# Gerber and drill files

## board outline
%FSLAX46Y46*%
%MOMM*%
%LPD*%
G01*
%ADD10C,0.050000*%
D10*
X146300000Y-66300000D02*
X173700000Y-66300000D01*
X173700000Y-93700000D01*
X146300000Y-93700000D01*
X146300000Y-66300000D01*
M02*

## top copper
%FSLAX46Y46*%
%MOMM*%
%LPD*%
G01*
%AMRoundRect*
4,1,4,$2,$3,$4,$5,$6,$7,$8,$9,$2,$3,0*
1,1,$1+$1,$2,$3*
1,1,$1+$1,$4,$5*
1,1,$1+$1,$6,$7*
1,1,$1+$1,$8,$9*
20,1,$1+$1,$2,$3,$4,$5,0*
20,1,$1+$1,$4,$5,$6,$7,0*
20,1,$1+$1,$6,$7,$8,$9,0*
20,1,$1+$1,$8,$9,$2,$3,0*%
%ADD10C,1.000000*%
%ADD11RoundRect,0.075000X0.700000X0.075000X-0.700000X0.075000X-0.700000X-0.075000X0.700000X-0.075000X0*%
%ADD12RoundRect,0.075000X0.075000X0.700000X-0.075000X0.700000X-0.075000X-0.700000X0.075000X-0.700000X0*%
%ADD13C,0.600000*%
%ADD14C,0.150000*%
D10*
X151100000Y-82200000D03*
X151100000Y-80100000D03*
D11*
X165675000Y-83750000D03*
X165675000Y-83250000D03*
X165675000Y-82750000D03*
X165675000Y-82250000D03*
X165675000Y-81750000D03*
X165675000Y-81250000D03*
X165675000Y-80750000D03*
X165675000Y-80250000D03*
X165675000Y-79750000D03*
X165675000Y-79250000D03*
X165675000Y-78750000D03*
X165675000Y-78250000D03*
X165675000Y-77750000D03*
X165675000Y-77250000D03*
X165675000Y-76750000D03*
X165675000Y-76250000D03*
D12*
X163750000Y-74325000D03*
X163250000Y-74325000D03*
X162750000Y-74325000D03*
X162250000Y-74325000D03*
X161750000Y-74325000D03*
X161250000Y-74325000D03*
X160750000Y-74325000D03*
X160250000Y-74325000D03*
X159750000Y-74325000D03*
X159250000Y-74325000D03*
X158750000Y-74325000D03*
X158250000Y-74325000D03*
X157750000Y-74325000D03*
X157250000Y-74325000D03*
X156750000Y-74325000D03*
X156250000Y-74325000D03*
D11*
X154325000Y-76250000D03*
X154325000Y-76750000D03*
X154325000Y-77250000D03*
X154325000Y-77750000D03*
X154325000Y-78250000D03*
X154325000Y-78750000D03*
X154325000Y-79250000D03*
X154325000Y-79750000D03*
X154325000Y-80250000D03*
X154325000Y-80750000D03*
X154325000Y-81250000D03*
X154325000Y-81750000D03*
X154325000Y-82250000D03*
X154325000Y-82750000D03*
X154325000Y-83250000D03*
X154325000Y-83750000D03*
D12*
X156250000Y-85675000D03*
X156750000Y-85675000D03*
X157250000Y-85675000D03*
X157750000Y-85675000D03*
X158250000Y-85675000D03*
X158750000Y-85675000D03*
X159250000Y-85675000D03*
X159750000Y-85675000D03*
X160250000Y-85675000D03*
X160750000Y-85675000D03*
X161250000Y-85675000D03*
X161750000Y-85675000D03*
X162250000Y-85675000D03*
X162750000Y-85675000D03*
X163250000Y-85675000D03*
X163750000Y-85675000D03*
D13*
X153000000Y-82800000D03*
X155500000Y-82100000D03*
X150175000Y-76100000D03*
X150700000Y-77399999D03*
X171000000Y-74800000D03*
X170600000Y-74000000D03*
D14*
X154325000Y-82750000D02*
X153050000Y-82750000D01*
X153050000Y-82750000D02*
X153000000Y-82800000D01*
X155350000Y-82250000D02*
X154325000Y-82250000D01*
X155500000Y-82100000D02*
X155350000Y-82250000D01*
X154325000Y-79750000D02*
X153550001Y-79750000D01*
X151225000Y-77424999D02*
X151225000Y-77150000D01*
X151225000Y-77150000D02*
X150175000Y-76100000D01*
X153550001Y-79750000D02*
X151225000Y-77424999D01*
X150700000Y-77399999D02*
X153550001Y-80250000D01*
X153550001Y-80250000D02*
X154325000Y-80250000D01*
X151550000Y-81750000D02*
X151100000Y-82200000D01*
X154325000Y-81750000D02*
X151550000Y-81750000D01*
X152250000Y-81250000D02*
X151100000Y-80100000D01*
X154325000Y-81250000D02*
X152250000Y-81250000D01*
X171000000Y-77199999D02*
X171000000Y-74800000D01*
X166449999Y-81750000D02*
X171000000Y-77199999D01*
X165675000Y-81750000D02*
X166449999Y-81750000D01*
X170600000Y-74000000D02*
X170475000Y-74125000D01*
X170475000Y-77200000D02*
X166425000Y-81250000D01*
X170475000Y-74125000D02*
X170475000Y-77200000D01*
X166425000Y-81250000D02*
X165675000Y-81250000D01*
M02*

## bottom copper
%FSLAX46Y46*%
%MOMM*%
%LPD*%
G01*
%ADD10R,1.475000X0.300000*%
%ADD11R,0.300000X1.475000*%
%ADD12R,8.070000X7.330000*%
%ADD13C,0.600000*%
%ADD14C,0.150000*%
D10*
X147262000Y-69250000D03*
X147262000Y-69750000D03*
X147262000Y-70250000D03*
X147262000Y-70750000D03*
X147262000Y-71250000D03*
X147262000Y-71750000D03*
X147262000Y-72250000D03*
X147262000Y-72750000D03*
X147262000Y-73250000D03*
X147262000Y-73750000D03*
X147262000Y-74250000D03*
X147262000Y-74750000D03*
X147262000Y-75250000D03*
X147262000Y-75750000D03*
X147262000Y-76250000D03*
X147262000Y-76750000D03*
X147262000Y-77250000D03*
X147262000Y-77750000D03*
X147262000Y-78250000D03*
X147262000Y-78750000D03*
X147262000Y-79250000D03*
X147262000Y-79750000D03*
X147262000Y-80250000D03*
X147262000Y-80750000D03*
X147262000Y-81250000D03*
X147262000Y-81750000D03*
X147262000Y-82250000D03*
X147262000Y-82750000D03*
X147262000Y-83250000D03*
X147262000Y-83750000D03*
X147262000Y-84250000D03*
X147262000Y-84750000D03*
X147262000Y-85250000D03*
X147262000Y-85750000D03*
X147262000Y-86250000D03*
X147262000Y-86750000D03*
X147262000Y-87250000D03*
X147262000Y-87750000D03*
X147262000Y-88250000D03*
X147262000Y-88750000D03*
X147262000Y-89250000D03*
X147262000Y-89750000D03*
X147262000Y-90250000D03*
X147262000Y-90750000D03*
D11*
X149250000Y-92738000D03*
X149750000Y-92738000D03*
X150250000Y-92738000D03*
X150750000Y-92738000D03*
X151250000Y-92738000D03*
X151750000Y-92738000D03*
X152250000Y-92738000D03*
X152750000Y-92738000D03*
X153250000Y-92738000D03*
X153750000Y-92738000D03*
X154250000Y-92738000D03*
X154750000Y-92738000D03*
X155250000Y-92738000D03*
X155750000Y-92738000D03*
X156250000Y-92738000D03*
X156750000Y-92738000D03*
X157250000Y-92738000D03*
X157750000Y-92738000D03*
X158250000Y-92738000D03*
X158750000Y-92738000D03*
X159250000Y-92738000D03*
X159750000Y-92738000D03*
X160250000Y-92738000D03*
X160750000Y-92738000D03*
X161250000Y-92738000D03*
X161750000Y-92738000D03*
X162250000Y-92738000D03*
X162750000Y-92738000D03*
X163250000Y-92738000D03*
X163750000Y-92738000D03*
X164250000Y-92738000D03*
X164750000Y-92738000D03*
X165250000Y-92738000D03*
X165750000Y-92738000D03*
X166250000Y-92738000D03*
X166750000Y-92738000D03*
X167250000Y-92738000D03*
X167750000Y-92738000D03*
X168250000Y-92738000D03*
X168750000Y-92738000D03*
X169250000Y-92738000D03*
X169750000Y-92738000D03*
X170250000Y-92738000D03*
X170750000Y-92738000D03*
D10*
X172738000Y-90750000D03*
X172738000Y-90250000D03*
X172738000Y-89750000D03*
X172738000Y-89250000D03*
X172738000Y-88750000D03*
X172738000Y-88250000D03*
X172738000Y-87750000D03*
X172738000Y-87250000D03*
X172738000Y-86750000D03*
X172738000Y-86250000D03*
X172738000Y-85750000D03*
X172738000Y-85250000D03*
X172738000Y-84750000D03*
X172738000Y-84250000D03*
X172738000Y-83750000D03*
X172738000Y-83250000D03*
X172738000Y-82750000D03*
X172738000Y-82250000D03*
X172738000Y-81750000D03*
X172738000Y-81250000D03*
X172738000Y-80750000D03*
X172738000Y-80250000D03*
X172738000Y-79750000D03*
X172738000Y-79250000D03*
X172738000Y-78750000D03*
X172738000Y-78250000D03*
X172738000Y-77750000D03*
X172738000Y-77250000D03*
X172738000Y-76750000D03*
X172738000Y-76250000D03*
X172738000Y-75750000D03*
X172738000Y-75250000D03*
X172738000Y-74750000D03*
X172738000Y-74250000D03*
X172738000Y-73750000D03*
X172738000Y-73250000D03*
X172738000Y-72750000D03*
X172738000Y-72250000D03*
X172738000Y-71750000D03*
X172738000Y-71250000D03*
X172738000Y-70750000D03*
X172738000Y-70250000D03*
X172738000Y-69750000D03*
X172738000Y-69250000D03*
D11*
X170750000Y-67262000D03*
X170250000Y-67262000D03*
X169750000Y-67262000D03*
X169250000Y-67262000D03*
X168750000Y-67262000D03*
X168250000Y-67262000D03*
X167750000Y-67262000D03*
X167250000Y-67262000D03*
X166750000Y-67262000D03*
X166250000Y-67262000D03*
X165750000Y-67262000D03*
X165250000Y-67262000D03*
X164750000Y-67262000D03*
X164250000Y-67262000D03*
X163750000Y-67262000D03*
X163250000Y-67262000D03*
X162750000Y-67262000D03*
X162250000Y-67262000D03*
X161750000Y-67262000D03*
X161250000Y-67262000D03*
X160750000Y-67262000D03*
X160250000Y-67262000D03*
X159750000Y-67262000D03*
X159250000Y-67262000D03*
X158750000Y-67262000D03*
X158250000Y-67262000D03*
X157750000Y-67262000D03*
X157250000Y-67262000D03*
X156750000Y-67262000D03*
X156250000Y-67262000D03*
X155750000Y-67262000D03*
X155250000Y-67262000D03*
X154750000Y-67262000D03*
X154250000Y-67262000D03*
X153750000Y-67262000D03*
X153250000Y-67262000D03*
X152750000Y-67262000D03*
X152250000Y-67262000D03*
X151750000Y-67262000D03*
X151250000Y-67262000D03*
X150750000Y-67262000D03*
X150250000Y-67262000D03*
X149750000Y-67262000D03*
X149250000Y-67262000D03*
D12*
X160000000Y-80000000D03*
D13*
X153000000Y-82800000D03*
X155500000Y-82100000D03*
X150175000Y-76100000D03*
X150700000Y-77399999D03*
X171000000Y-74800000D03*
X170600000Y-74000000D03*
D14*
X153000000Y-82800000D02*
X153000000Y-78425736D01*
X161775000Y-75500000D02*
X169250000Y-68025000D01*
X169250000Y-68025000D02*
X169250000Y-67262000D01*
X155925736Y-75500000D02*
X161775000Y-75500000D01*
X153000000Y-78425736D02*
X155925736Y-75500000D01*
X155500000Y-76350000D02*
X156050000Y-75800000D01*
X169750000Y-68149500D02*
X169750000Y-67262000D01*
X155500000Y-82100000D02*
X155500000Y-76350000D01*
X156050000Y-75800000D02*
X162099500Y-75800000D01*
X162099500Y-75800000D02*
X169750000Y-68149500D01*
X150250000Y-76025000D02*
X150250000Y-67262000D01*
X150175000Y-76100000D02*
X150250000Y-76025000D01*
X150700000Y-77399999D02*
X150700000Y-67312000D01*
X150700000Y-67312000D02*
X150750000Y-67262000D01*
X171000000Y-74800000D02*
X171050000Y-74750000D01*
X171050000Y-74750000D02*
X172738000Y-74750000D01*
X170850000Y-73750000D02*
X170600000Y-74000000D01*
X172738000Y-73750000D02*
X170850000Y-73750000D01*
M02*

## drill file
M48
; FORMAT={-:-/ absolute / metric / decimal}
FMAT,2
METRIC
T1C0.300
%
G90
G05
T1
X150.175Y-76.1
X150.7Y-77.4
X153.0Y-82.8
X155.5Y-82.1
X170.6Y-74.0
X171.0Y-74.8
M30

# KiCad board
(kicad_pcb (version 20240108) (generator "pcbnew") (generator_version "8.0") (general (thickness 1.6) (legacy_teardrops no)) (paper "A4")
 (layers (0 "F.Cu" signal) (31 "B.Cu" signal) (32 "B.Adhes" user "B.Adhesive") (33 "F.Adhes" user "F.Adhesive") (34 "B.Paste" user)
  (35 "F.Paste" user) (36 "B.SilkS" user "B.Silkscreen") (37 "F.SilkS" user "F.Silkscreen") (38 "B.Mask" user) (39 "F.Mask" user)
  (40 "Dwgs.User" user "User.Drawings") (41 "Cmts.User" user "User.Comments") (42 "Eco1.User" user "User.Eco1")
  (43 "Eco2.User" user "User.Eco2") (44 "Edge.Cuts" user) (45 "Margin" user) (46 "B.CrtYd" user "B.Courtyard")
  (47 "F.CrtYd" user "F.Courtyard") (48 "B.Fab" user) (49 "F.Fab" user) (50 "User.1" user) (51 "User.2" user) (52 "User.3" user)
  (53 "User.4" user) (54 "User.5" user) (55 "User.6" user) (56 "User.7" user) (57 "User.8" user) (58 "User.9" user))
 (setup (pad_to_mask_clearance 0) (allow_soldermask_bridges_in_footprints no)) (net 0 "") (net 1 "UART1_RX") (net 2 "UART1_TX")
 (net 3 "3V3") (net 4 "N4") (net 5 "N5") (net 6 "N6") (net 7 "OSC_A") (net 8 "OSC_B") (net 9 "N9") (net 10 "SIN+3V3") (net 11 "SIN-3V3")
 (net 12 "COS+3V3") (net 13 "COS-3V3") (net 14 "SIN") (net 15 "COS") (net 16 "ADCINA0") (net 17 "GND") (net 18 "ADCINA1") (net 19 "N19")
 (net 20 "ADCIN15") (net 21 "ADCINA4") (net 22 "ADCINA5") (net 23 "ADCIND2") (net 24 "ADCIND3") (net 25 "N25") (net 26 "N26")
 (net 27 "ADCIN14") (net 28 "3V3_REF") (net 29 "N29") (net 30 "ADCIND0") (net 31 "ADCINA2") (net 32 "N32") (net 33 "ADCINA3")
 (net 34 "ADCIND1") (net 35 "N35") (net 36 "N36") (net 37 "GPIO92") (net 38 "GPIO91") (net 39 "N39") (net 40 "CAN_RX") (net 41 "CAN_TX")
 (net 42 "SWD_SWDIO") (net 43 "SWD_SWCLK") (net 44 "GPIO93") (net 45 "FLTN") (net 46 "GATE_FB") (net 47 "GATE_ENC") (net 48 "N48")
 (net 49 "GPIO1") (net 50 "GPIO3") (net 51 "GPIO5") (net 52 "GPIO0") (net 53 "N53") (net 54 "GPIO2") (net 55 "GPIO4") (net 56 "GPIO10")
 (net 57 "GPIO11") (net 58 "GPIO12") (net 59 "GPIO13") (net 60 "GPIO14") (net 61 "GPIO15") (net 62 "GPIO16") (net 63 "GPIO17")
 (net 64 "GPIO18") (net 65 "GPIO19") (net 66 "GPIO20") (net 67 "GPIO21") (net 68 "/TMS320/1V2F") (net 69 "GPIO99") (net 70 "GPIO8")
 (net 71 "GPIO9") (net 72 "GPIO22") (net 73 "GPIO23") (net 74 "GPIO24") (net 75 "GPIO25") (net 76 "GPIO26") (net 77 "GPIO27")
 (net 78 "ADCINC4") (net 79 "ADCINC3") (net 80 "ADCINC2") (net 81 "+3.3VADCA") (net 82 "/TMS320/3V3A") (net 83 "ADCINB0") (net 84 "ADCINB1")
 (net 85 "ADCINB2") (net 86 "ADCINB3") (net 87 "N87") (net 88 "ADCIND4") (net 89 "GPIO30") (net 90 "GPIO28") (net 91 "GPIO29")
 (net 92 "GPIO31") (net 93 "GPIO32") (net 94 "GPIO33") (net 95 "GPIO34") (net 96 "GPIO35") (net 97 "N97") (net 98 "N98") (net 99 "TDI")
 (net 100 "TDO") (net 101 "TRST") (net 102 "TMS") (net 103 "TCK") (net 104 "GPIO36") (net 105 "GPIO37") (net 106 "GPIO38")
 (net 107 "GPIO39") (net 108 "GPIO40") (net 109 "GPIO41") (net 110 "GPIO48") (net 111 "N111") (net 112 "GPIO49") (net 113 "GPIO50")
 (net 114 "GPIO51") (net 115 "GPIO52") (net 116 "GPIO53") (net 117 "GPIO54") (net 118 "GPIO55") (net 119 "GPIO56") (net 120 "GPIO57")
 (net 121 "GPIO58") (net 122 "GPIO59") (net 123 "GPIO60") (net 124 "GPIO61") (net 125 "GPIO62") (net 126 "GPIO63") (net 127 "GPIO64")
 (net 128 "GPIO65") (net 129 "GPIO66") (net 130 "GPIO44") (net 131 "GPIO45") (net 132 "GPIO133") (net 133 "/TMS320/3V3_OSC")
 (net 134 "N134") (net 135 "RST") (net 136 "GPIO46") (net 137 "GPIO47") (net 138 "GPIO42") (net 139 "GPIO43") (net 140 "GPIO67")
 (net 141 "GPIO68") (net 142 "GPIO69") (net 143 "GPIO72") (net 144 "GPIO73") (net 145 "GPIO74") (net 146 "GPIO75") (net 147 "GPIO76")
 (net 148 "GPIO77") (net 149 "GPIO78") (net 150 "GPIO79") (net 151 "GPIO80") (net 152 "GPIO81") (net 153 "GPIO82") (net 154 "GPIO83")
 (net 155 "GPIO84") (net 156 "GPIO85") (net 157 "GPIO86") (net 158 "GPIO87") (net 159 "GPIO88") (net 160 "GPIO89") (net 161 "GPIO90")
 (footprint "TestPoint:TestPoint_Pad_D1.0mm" (layer "F.Cu") (at 151.1 82.2)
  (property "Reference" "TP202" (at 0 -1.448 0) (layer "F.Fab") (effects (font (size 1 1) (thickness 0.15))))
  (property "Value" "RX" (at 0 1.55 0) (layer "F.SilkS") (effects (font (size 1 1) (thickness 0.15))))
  (pad "1" smd circle (at 0 0) (size 1 1) (layers "F.Cu" "F.Mask") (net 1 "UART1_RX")))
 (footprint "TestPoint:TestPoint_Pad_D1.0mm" (layer "F.Cu") (at 151.1 80.1)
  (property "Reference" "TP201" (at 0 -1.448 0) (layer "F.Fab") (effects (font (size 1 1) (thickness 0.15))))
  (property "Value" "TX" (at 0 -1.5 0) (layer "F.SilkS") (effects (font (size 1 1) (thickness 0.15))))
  (pad "1" smd circle (at 0 0) (size 1 1) (layers "F.Cu" "F.Mask") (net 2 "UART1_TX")))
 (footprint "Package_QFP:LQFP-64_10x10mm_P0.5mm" (layer "F.Cu") (at 160 80 180)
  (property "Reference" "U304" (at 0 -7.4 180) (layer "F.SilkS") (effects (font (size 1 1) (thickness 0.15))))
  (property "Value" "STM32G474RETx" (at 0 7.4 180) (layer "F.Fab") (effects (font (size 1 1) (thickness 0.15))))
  (pad "1" smd roundrect (at -5.675 -3.75 180) (size 1.55 0.3) (layers "F.Cu" "F.Paste" "F.Mask") (roundrect_rratio 0.25) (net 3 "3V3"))
  (pad "2" smd roundrect (at -5.675 -3.25 180) (size 1.55 0.3) (layers "F.Cu" "F.Paste" "F.Mask") (roundrect_rratio 0.25) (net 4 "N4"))
  (pad "3" smd roundrect (at -5.675 -2.75 180) (size 1.55 0.3) (layers "F.Cu" "F.Paste" "F.Mask") (roundrect_rratio 0.25) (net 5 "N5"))
  (pad "4" smd roundrect (at -5.675 -2.25 180) (size 1.55 0.3) (layers "F.Cu" "F.Paste" "F.Mask") (roundrect_rratio 0.25) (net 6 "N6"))
  (pad "5" smd roundrect (at -5.675 -1.75 180) (size 1.55 0.3) (layers "F.Cu" "F.Paste" "F.Mask") (roundrect_rratio 0.25) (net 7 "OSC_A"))
  (pad "6" smd roundrect (at -5.675 -1.25 180) (size 1.55 0.3) (layers "F.Cu" "F.Paste" "F.Mask") (roundrect_rratio 0.25) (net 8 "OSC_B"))
  (pad "7" smd roundrect (at -5.675 -0.75 180) (size 1.55 0.3) (layers "F.Cu" "F.Paste" "F.Mask") (roundrect_rratio 0.25) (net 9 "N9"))
  (pad "8" smd roundrect (at -5.675 -0.25 180) (size 1.55 0.3) (layers "F.Cu" "F.Paste" "F.Mask") (roundrect_rratio 0.25) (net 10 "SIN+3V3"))
  (pad "9" smd roundrect (at -5.675 0.25 180) (size 1.55 0.3) (layers "F.Cu" "F.Paste" "F.Mask") (roundrect_rratio 0.25) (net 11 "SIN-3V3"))
  (pad "10" smd roundrect (at -5.675 0.75 180) (size 1.55 0.3) (layers "F.Cu" "F.Paste" "F.Mask") (roundrect_rratio 0.25) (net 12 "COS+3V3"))
  (pad "11" smd roundrect (at -5.675 1.25 180) (size 1.55 0.3) (layers "F.Cu" "F.Paste" "F.Mask") (roundrect_rratio 0.25) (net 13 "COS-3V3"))
  (pad "12" smd roundrect (at -5.675 1.75 180) (size 1.55 0.3) (layers "F.Cu" "F.Paste" "F.Mask") (roundrect_rratio 0.25) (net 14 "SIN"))
  (pad "13" smd roundrect (at -5.675 2.25 180) (size 1.55 0.3) (layers "F.Cu" "F.Paste" "F.Mask") (roundrect_rratio 0.25) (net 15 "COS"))
  (pad "14" smd roundrect (at -5.675 2.75 180) (size 1.55 0.3) (layers "F.Cu" "F.Paste" "F.Mask") (roundrect_rratio 0.25) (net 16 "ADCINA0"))
  (pad "15" smd roundrect (at -5.675 3.25 180) (size 1.55 0.3) (layers "F.Cu" "F.Paste" "F.Mask") (roundrect_rratio 0.25) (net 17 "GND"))
  (pad "16" smd roundrect (at -5.675 3.75 180) (size 1.55 0.3) (layers "F.Cu" "F.Paste" "F.Mask") (roundrect_rratio 0.25) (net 3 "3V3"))
  (pad "17" smd roundrect (at -3.75 5.675 180) (size 0.3 1.55) (layers "F.Cu" "F.Paste" "F.Mask") (roundrect_rratio 0.25) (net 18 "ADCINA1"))
  (pad "18" smd roundrect (at -3.25 5.675 180) (size 0.3 1.55) (layers "F.Cu" "F.Paste" "F.Mask") (roundrect_rratio 0.25) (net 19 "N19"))
  (pad "19" smd roundrect (at -2.75 5.675 180) (size 0.3 1.55) (layers "F.Cu" "F.Paste" "F.Mask") (roundrect_rratio 0.25) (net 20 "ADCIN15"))
  (pad "20" smd roundrect (at -2.25 5.675 180) (size 0.3 1.55) (layers "F.Cu" "F.Paste" "F.Mask") (roundrect_rratio 0.25) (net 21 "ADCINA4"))
  (pad "21" smd roundrect (at -1.75 5.675 180) (size 0.3 1.55) (layers "F.Cu" "F.Paste" "F.Mask") (roundrect_rratio 0.25) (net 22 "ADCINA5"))
  (pad "22" smd roundrect (at -1.25 5.675 180) (size 0.3 1.55) (layers "F.Cu" "F.Paste" "F.Mask") (roundrect_rratio 0.25) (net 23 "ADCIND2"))
  (pad "23" smd roundrect (at -0.75 5.675 180) (size 0.3 1.55) (layers "F.Cu" "F.Paste" "F.Mask") (roundrect_rratio 0.25) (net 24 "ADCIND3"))
  (pad "24" smd roundrect (at -0.25 5.675 180) (size 0.3 1.55) (layers "F.Cu" "F.Paste" "F.Mask") (roundrect_rratio 0.25) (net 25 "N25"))
  (pad "25" smd roundrect (at 0.25 5.675 180) (size 0.3 1.55) (layers "F.Cu" "F.Paste" "F.Mask") (roundrect_rratio 0.25) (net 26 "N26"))
  (pad "26" smd roundrect (at 0.75 5.675 180) (size 0.3 1.55) (layers "F.Cu" "F.Paste" "F.Mask") (roundrect_rratio 0.25) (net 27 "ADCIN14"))
  (pad "27" smd roundrect (at 1.25 5.675 180) (size 0.3 1.55) (layers "F.Cu" "F.Paste" "F.Mask") (roundrect_rratio 0.25) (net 17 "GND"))
  (pad "28" smd roundrect (at 1.75 5.675 180) (size 0.3 1.55) (layers "F.Cu" "F.Paste" "F.Mask") (roundrect_rratio 0.25) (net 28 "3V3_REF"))
  (pad "29" smd roundrect (at 2.25 5.675 180) (size 0.3 1.55) (layers "F.Cu" "F.Paste" "F.Mask") (roundrect_rratio 0.25) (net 3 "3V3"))
  (pad "30" smd roundrect (at 2.75 5.675 180) (size 0.3 1.55) (layers "F.Cu" "F.Paste" "F.Mask") (roundrect_rratio 0.25) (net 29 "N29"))
  (pad "31" smd roundrect (at 3.25 5.675 180) (size 0.3 1.55) (layers "F.Cu" "F.Paste" "F.Mask") (roundrect_rratio 0.25) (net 17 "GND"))
  (pad "32" smd roundrect (at 3.75 5.675 180) (size 0.3 1.55) (layers "F.Cu" "F.Paste" "F.Mask") (roundrect_rratio 0.25) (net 3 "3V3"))
  (pad "33" smd roundrect (at 5.675 3.75 180) (size 1.55 0.3) (layers "F.Cu" "F.Paste" "F.Mask") (roundrect_rratio 0.25) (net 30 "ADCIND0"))
  (pad "34" smd roundrect (at 5.675 3.25 180) (size 1.55 0.3) (layers "F.Cu" "F.Paste" "F.Mask") (roundrect_rratio 0.25) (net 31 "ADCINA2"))
  (pad "35" smd roundrect (at 5.675 2.75 180) (size 1.55 0.3) (layers "F.Cu" "F.Paste" "F.Mask") (roundrect_rratio 0.25) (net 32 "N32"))
  (pad "36" smd roundrect (at 5.675 2.25 180) (size 1.55 0.3) (layers "F.Cu" "F.Paste" "F.Mask") (roundrect_rratio 0.25) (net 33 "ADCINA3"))
  (pad "37" smd roundrect (at 5.675 1.75 180) (size 1.55 0.3) (layers "F.Cu" "F.Paste" "F.Mask") (roundrect_rratio 0.25) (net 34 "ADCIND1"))
  (pad "38" smd roundrect (at 5.675 1.25 180) (size 1.55 0.3) (layers "F.Cu" "F.Paste" "F.Mask") (roundrect_rratio 0.25) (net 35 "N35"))
  (pad "39" smd roundrect (at 5.675 0.75 180) (size 1.55 0.3) (layers "F.Cu" "F.Paste" "F.Mask") (roundrect_rratio 0.25) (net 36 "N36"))
  (pad "40" smd roundrect (at 5.675 0.25 180) (size 1.55 0.3) (layers "F.Cu" "F.Paste" "F.Mask") (roundrect_rratio 0.25) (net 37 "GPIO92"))
  (pad "41" smd roundrect (at 5.675 -0.25 180) (size 1.55 0.3) (layers "F.Cu" "F.Paste" "F.Mask") (roundrect_rratio 0.25) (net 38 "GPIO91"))
  (pad "42" smd roundrect (at 5.675 -0.75 180) (size 1.55 0.3) (layers "F.Cu" "F.Paste" "F.Mask") (roundrect_rratio 0.25) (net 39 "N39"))
  (pad "43" smd roundrect (at 5.675 -1.25 180) (size 1.55 0.3) (layers "F.Cu" "F.Paste" "F.Mask") (roundrect_rratio 0.25) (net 2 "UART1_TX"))
  (pad "44" smd roundrect (at 5.675 -1.75 180) (size 1.55 0.3) (layers "F.Cu" "F.Paste" "F.Mask") (roundrect_rratio 0.25) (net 1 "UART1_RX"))
  (pad "45" smd roundrect (at 5.675 -2.25 180) (size 1.55 0.3) (layers "F.Cu" "F.Paste" "F.Mask") (roundrect_rratio 0.25) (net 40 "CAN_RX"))
  (pad "46" smd roundrect (at 5.675 -2.75 180) (size 1.55 0.3) (layers "F.Cu" "F.Paste" "F.Mask") (roundrect_rratio 0.25) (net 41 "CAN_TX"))
  (pad "47" smd roundrect (at 5.675 -3.25 180) (size 1.55 0.3) (layers "F.Cu" "F.Paste" "F.Mask") (roundrect_rratio 0.25) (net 17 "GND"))
  (pad "48" smd roundrect (at 5.675 -3.75 180) (size 1.55 0.3) (layers "F.Cu" "F.Paste" "F.Mask") (roundrect_rratio 0.25) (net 3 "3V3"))
  (pad "49" smd roundrect (at 3.75 -5.675 180) (size 0.3 1.55) (layers "F.Cu" "F.Paste" "F.Mask") (roundrect_rratio 0.25)
   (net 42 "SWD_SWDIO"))
  (pad "50" smd roundrect (at 3.25 -5.675 180) (size 0.3 1.55) (layers "F.Cu" "F.Paste" "F.Mask") (roundrect_rratio 0.25)
   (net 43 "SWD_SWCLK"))
  (pad "51" smd roundrect (at 2.75 -5.675 180) (size 0.3 1.55) (layers "F.Cu" "F.Paste" "F.Mask") (roundrect_rratio 0.25) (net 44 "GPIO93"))
  (pad "52" smd roundrect (at 2.25 -5.675 180) (size 0.3 1.55) (layers "F.Cu" "F.Paste" "F.Mask") (roundrect_rratio 0.25) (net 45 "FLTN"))
  (pad "53" smd roundrect (at 1.75 -5.675 180) (size 0.3 1.55) (layers "F.Cu" "F.Paste" "F.Mask") (roundrect_rratio 0.25) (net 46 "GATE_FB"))
  (pad "54" smd roundrect (at 1.25 -5.675 180) (size 0.3 1.55) (layers "F.Cu" "F.Paste" "F.Mask") (roundrect_rratio 0.25)
   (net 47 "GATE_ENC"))
  (pad "55" smd roundrect (at 0.75 -5.675 180) (size 0.3 1.55) (layers "F.Cu" "F.Paste" "F.Mask") (roundrect_rratio 0.25) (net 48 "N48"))
  (pad "56" smd roundrect (at 0.25 -5.675 180) (size 0.3 1.55) (layers "F.Cu" "F.Paste" "F.Mask") (roundrect_rratio 0.25) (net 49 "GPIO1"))
  (pad "57" smd roundrect (at -0.25 -5.675 180) (size 0.3 1.55) (layers "F.Cu" "F.Paste" "F.Mask") (roundrect_rratio 0.25) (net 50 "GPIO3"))
  (pad "58" smd roundrect (at -0.75 -5.675 180) (size 0.3 1.55) (layers "F.Cu" "F.Paste" "F.Mask") (roundrect_rratio 0.25) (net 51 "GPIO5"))
  (pad "59" smd roundrect (at -1.25 -5.675 180) (size 0.3 1.55) (layers "F.Cu" "F.Paste" "F.Mask") (roundrect_rratio 0.25) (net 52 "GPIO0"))
  (pad "60" smd roundrect (at -1.75 -5.675 180) (size 0.3 1.55) (layers "F.Cu" "F.Paste" "F.Mask") (roundrect_rratio 0.25) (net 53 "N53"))
  (pad "61" smd roundrect (at -2.25 -5.675 180) (size 0.3 1.55) (layers "F.Cu" "F.Paste" "F.Mask") (roundrect_rratio 0.25) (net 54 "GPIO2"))
  (pad "62" smd roundrect (at -2.75 -5.675 180) (size 0.3 1.55) (layers "F.Cu" "F.Paste" "F.Mask") (roundrect_rratio 0.25) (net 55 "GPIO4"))
  (pad "63" smd roundrect (at -3.25 -5.675 180) (size 0.3 1.55) (layers "F.Cu" "F.Paste" "F.Mask") (roundrect_rratio 0.25) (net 17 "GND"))
  (pad "64" smd roundrect (at -3.75 -5.675 180) (size 0.3 1.55) (layers "F.Cu" "F.Paste" "F.Mask") (roundrect_rratio 0.25) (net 3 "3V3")))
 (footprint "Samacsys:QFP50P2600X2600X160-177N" (layer "B.Cu") (at 160 80 180)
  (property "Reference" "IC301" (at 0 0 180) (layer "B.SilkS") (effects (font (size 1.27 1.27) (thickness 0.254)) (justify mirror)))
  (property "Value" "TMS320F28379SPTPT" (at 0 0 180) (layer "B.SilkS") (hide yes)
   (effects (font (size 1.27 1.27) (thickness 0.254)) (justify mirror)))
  (pad "1" smd rect (at 12.738 10.75 270) (size 0.3 1.475) (layers "B.Cu" "B.Paste" "B.Mask") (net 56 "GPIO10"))
  (pad "2" smd rect (at 12.738 10.25 270) (size 0.3 1.475) (layers "B.Cu" "B.Paste" "B.Mask") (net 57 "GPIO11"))
  (pad "3" smd rect (at 12.738 9.75 270) (size 0.3 1.475) (layers "B.Cu" "B.Paste" "B.Mask") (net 3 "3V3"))
  (pad "4" smd rect (at 12.738 9.25 270) (size 0.3 1.475) (layers "B.Cu" "B.Paste" "B.Mask") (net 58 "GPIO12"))
  (pad "5" smd rect (at 12.738 8.75 270) (size 0.3 1.475) (layers "B.Cu" "B.Paste" "B.Mask") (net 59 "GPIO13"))
  (pad "6" smd rect (at 12.738 8.25 270) (size 0.3 1.475) (layers "B.Cu" "B.Paste" "B.Mask") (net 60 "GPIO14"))
  (pad "7" smd rect (at 12.738 7.75 270) (size 0.3 1.475) (layers "B.Cu" "B.Paste" "B.Mask") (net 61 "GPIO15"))
  (pad "8" smd rect (at 12.738 7.25 270) (size 0.3 1.475) (layers "B.Cu" "B.Paste" "B.Mask") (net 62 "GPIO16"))
  (pad "9" smd rect (at 12.738 6.75 270) (size 0.3 1.475) (layers "B.Cu" "B.Paste" "B.Mask") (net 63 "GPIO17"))
  (pad "10" smd rect (at 12.738 6.25 270) (size 0.3 1.475) (layers "B.Cu" "B.Paste" "B.Mask") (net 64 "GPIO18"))
  (pad "11" smd rect (at 12.738 5.75 270) (size 0.3 1.475) (layers "B.Cu" "B.Paste" "B.Mask") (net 3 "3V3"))
  (pad "12" smd rect (at 12.738 5.25 270) (size 0.3 1.475) (layers "B.Cu" "B.Paste" "B.Mask") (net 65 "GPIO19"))
  (pad "13" smd rect (at 12.738 4.75 270) (size 0.3 1.475) (layers "B.Cu" "B.Paste" "B.Mask") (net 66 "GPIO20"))
  (pad "14" smd rect (at 12.738 4.25 270) (size 0.3 1.475) (layers "B.Cu" "B.Paste" "B.Mask") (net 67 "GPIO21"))
  (pad "15" smd rect (at 12.738 3.75 270) (size 0.3 1.475) (layers "B.Cu" "B.Paste" "B.Mask") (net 3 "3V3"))
  (pad "16" smd rect (at 12.738 3.25 270) (size 0.3 1.475) (layers "B.Cu" "B.Paste" "B.Mask") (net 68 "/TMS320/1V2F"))
  (pad "17" smd rect (at 12.738 2.75 270) (size 0.3 1.475) (layers "B.Cu" "B.Paste" "B.Mask") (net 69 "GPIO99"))
  (pad "18" smd rect (at 12.738 2.25 270) (size 0.3 1.475) (layers "B.Cu" "B.Paste" "B.Mask") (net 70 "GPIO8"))
  (pad "19" smd rect (at 12.738 1.75 270) (size 0.3 1.475) (layers "B.Cu" "B.Paste" "B.Mask") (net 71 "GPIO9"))
  (pad "20" smd rect (at 12.738 1.25 270) (size 0.3 1.475) (layers "B.Cu" "B.Paste" "B.Mask") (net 3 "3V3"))
  (pad "21" smd rect (at 12.738 0.75 270) (size 0.3 1.475) (layers "B.Cu" "B.Paste" "B.Mask") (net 68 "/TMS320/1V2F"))
  (pad "22" smd rect (at 12.738 0.25 270) (size 0.3 1.475) (layers "B.Cu" "B.Paste" "B.Mask") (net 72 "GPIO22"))
  (pad "23" smd rect (at 12.738 -0.25 270) (size 0.3 1.475) (layers "B.Cu" "B.Paste" "B.Mask") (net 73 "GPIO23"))
  (pad "24" smd rect (at 12.738 -0.75 270) (size 0.3 1.475) (layers "B.Cu" "B.Paste" "B.Mask") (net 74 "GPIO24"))
  (pad "25" smd rect (at 12.738 -1.25 270) (size 0.3 1.475) (layers "B.Cu" "B.Paste" "B.Mask") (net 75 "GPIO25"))
  (pad "26" smd rect (at 12.738 -1.75 270) (size 0.3 1.475) (layers "B.Cu" "B.Paste" "B.Mask") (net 3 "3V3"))
  (pad "27" smd rect (at 12.738 -2.25 270) (size 0.3 1.475) (layers "B.Cu" "B.Paste" "B.Mask") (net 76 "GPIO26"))
  (pad "28" smd rect (at 12.738 -2.75 270) (size 0.3 1.475) (layers "B.Cu" "B.Paste" "B.Mask") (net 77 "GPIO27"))
  (pad "29" smd rect (at 12.738 -3.25 270) (size 0.3 1.475) (layers "B.Cu" "B.Paste" "B.Mask") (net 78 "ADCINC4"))
  (pad "30" smd rect (at 12.738 -3.75 270) (size 0.3 1.475) (layers "B.Cu" "B.Paste" "B.Mask") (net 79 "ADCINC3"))
  (pad "31" smd rect (at 12.738 -4.25 270) (size 0.3 1.475) (layers "B.Cu" "B.Paste" "B.Mask") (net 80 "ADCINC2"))
  (pad "32" smd rect (at 12.738 -4.75 270) (size 0.3 1.475) (layers "B.Cu" "B.Paste" "B.Mask") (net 17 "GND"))
  (pad "33" smd rect (at 12.738 -5.25 270) (size 0.3 1.475) (layers "B.Cu" "B.Paste" "B.Mask") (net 17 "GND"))
  (pad "34" smd rect (at 12.738 -5.75 270) (size 0.3 1.475) (layers "B.Cu" "B.Paste" "B.Mask") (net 17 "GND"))
  (pad "35" smd rect (at 12.738 -6.25 270) (size 0.3 1.475) (layers "B.Cu" "B.Paste" "B.Mask") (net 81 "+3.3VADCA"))
  (pad "36" smd rect (at 12.738 -6.75 270) (size 0.3 1.475) (layers "B.Cu" "B.Paste" "B.Mask") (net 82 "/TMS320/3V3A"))
  (pad "37" smd rect (at 12.738 -7.25 270) (size 0.3 1.475) (layers "B.Cu" "B.Paste" "B.Mask") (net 81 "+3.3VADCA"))
  (pad "38" smd rect (at 12.738 -7.75 270) (size 0.3 1.475) (layers "B.Cu" "B.Paste" "B.Mask") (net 22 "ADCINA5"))
  (pad "39" smd rect (at 12.738 -8.25 270) (size 0.3 1.475) (layers "B.Cu" "B.Paste" "B.Mask") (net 21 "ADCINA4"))
  (pad "40" smd rect (at 12.738 -8.75 270) (size 0.3 1.475) (layers "B.Cu" "B.Paste" "B.Mask") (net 33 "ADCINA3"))
  (pad "41" smd rect (at 12.738 -9.25 270) (size 0.3 1.475) (layers "B.Cu" "B.Paste" "B.Mask") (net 31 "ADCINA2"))
  (pad "42" smd rect (at 12.738 -9.75 270) (size 0.3 1.475) (layers "B.Cu" "B.Paste" "B.Mask") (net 18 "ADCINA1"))
  (pad "43" smd rect (at 12.738 -10.25 270) (size 0.3 1.475) (layers "B.Cu" "B.Paste" "B.Mask") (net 16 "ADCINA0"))
  (pad "44" smd rect (at 12.738 -10.75 270) (size 0.3 1.475) (layers "B.Cu" "B.Paste" "B.Mask") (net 27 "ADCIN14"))
  (pad "45" smd rect (at 10.75 -12.738 180) (size 0.3 1.475) (layers "B.Cu" "B.Paste" "B.Mask") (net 20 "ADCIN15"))
  (pad "46" smd rect (at 10.25 -12.738 180) (size 0.3 1.475) (layers "B.Cu" "B.Paste" "B.Mask") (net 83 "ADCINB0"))
  (pad "47" smd rect (at 9.75 -12.738 180) (size 0.3 1.475) (layers "B.Cu" "B.Paste" "B.Mask") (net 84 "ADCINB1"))
  (pad "48" smd rect (at 9.25 -12.738 180) (size 0.3 1.475) (layers "B.Cu" "B.Paste" "B.Mask") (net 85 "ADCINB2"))
  (pad "49" smd rect (at 8.75 -12.738 180) (size 0.3 1.475) (layers "B.Cu" "B.Paste" "B.Mask") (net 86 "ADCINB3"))
  (pad "50" smd rect (at 8.25 -12.738 180) (size 0.3 1.475) (layers "B.Cu" "B.Paste" "B.Mask") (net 17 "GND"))
  (pad "51" smd rect (at 7.75 -12.738 180) (size 0.3 1.475) (layers "B.Cu" "B.Paste" "B.Mask") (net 17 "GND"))
  (pad "52" smd rect (at 7.25 -12.738 180) (size 0.3 1.475) (layers "B.Cu" "B.Paste" "B.Mask") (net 17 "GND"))
  (pad "53" smd rect (at 6.75 -12.738 180) (size 0.3 1.475) (layers "B.Cu" "B.Paste" "B.Mask") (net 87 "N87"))
  (pad "54" smd rect (at 6.25 -12.738 180) (size 0.3 1.475) (layers "B.Cu" "B.Paste" "B.Mask") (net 82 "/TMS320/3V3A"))
  (pad "55" smd rect (at 5.75 -12.738 180) (size 0.3 1.475) (layers "B.Cu" "B.Paste" "B.Mask") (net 87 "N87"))
  (pad "56" smd rect (at 5.25 -12.738 180) (size 0.3 1.475) (layers "B.Cu" "B.Paste" "B.Mask") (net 30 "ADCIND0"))
  (pad "57" smd rect (at 4.75 -12.738 180) (size 0.3 1.475) (layers "B.Cu" "B.Paste" "B.Mask") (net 34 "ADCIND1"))
  (pad "58" smd rect (at 4.25 -12.738 180) (size 0.3 1.475) (layers "B.Cu" "B.Paste" "B.Mask") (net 23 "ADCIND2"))
  (pad "59" smd rect (at 3.75 -12.738 180) (size 0.3 1.475) (layers "B.Cu" "B.Paste" "B.Mask") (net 24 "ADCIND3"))
  (pad "60" smd rect (at 3.25 -12.738 180) (size 0.3 1.475) (layers "B.Cu" "B.Paste" "B.Mask") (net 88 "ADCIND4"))
  (pad "61" smd rect (at 2.75 -12.738 180) (size 0.3 1.475) (layers "B.Cu" "B.Paste" "B.Mask") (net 68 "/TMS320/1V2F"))
  (pad "62" smd rect (at 2.25 -12.738 180) (size 0.3 1.475) (layers "B.Cu" "B.Paste" "B.Mask") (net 3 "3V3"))
  (pad "63" smd rect (at 1.75 -12.738 180) (size 0.3 1.475) (layers "B.Cu" "B.Paste" "B.Mask") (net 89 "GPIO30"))
  (pad "64" smd rect (at 1.25 -12.738 180) (size 0.3 1.475) (layers "B.Cu" "B.Paste" "B.Mask") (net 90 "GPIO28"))
  (pad "65" smd rect (at 0.75 -12.738 180) (size 0.3 1.475) (layers "B.Cu" "B.Paste" "B.Mask") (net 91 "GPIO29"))
  (pad "66" smd rect (at 0.25 -12.738 180) (size 0.3 1.475) (layers "B.Cu" "B.Paste" "B.Mask") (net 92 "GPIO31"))
  (pad "67" smd rect (at -0.25 -12.738 180) (size 0.3 1.475) (layers "B.Cu" "B.Paste" "B.Mask") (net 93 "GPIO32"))
  (pad "68" smd rect (at -0.75 -12.738 180) (size 0.3 1.475) (layers "B.Cu" "B.Paste" "B.Mask") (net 3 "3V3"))
  (pad "69" smd rect (at -1.25 -12.738 180) (size 0.3 1.475) (layers "B.Cu" "B.Paste" "B.Mask") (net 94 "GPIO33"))
  (pad "70" smd rect (at -1.75 -12.738 180) (size 0.3 1.475) (layers "B.Cu" "B.Paste" "B.Mask") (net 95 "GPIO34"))
  (pad "71" smd rect (at -2.25 -12.738 180) (size 0.3 1.475) (layers "B.Cu" "B.Paste" "B.Mask") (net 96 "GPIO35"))
  (pad "72" smd rect (at -2.75 -12.738 180) (size 0.3 1.475) (layers "B.Cu" "B.Paste" "B.Mask") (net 3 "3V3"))
  (pad "73" smd rect (at -3.25 -12.738 180) (size 0.3 1.475) (layers "B.Cu" "B.Paste" "B.Mask") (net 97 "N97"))
  (pad "74" smd rect (at -3.75 -12.738 180) (size 0.3 1.475) (layers "B.Cu" "B.Paste" "B.Mask") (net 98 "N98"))
  (pad "75" smd rect (at -4.25 -12.738 180) (size 0.3 1.475) (layers "B.Cu" "B.Paste" "B.Mask") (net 3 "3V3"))
  (pad "76" smd rect (at -4.75 -12.738 180) (size 0.3 1.475) (layers "B.Cu" "B.Paste" "B.Mask") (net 68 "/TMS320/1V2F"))
  (pad "77" smd rect (at -5.25 -12.738 180) (size 0.3 1.475) (layers "B.Cu" "B.Paste" "B.Mask") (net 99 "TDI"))
  (pad "78" smd rect (at -5.75 -12.738 180) (size 0.3 1.475) (layers "B.Cu" "B.Paste" "B.Mask") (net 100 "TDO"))
  (pad "79" smd rect (at -6.25 -12.738 180) (size 0.3 1.475) (layers "B.Cu" "B.Paste" "B.Mask") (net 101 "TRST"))
  (pad "80" smd rect (at -6.75 -12.738 180) (size 0.3 1.475) (layers "B.Cu" "B.Paste" "B.Mask") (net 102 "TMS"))
  (pad "81" smd rect (at -7.25 -12.738 180) (size 0.3 1.475) (layers "B.Cu" "B.Paste" "B.Mask") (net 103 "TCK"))
  (pad "82" smd rect (at -7.75 -12.738 180) (size 0.3 1.475) (layers "B.Cu" "B.Paste" "B.Mask") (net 3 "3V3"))
  (pad "83" smd rect (at -8.25 -12.738 180) (size 0.3 1.475) (layers "B.Cu" "B.Paste" "B.Mask") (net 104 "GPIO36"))
  (pad "84" smd rect (at -8.75 -12.738 180) (size 0.3 1.475) (layers "B.Cu" "B.Paste" "B.Mask") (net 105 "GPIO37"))
  (pad "85" smd rect (at -9.25 -12.738 180) (size 0.3 1.475) (layers "B.Cu" "B.Paste" "B.Mask") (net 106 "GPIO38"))
  (pad "86" smd rect (at -9.75 -12.738 180) (size 0.3 1.475) (layers "B.Cu" "B.Paste" "B.Mask") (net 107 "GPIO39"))
  (pad "87" smd rect (at -10.25 -12.738 180) (size 0.3 1.475) (layers "B.Cu" "B.Paste" "B.Mask") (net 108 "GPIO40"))
  (pad "88" smd rect (at -10.75 -12.738 180) (size 0.3 1.475) (layers "B.Cu" "B.Paste" "B.Mask") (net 3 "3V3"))
  (pad "89" smd rect (at -12.738 -10.75 270) (size 0.3 1.475) (layers "B.Cu" "B.Paste" "B.Mask") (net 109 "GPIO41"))
  (pad "90" smd rect (at -12.738 -10.25 270) (size 0.3 1.475) (layers "B.Cu" "B.Paste" "B.Mask") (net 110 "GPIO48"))
  (pad "91" smd rect (at -12.738 -9.75 270) (size 0.3 1.475) (layers "B.Cu" "B.Paste" "B.Mask") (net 3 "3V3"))
  (pad "92" smd rect (at -12.738 -9.25 270) (size 0.3 1.475) (layers "B.Cu" "B.Paste" "B.Mask") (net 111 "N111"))
  (pad "93" smd rect (at -12.738 -8.75 270) (size 0.3 1.475) (layers "B.Cu" "B.Paste" "B.Mask") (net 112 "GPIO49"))
  (pad "94" smd rect (at -12.738 -8.25 270) (size 0.3 1.475) (layers "B.Cu" "B.Paste" "B.Mask") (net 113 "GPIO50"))
  (pad "95" smd rect (at -12.738 -7.75 270) (size 0.3 1.475) (layers "B.Cu" "B.Paste" "B.Mask") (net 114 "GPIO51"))
  (pad "96" smd rect (at -12.738 -7.25 270) (size 0.3 1.475) (layers "B.Cu" "B.Paste" "B.Mask") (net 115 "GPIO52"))
  (pad "97" smd rect (at -12.738 -6.75 270) (size 0.3 1.475) (layers "B.Cu" "B.Paste" "B.Mask") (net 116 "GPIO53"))
  (pad "98" smd rect (at -12.738 -6.25 270) (size 0.3 1.475) (layers "B.Cu" "B.Paste" "B.Mask") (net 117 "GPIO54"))
  (pad "99" smd rect (at -12.738 -5.75 270) (size 0.3 1.475) (layers "B.Cu" "B.Paste" "B.Mask") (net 3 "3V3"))
  (pad "100" smd rect (at -12.738 -5.25 270) (size 0.3 1.475) (layers "B.Cu" "B.Paste" "B.Mask") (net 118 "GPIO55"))
  (pad "101" smd rect (at -12.738 -4.75 270) (size 0.3 1.475) (layers "B.Cu" "B.Paste" "B.Mask") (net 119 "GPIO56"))
  (pad "102" smd rect (at -12.738 -4.25 270) (size 0.3 1.475) (layers "B.Cu" "B.Paste" "B.Mask") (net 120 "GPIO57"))
  (pad "103" smd rect (at -12.738 -3.75 270) (size 0.3 1.475) (layers "B.Cu" "B.Paste" "B.Mask") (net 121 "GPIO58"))
  (pad "104" smd rect (at -12.738 -3.25 270) (size 0.3 1.475) (layers "B.Cu" "B.Paste" "B.Mask") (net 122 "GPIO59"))
  (pad "105" smd rect (at -12.738 -2.75 270) (size 0.3 1.475) (layers "B.Cu" "B.Paste" "B.Mask") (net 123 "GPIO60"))
  (pad "106" smd rect (at -12.738 -2.25 270) (size 0.3 1.475) (layers "B.Cu" "B.Paste" "B.Mask") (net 3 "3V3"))
  (pad "107" smd rect (at -12.738 -1.75 270) (size 0.3 1.475) (layers "B.Cu" "B.Paste" "B.Mask") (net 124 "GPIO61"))
  (pad "108" smd rect (at -12.738 -1.25 270) (size 0.3 1.475) (layers "B.Cu" "B.Paste" "B.Mask") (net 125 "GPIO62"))
  (pad "109" smd rect (at -12.738 -0.75 270) (size 0.3 1.475) (layers "B.Cu" "B.Paste" "B.Mask") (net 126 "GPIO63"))
  (pad "110" smd rect (at -12.738 -0.25 270) (size 0.3 1.475) (layers "B.Cu" "B.Paste" "B.Mask") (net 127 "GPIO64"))
  (pad "111" smd rect (at -12.738 0.25 270) (size 0.3 1.475) (layers "B.Cu" "B.Paste" "B.Mask") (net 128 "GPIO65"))
  (pad "112" smd rect (at -12.738 0.75 270) (size 0.3 1.475) (layers "B.Cu" "B.Paste" "B.Mask") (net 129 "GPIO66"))
  (pad "113" smd rect (at -12.738 1.25 270) (size 0.3 1.475) (layers "B.Cu" "B.Paste" "B.Mask") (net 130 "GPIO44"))
  (pad "114" smd rect (at -12.738 1.75 270) (size 0.3 1.475) (layers "B.Cu" "B.Paste" "B.Mask") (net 3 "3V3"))
  (pad "115" smd rect (at -12.738 2.25 270) (size 0.3 1.475) (layers "B.Cu" "B.Paste" "B.Mask") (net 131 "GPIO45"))
  (pad "116" smd rect (at -12.738 2.75 270) (size 0.3 1.475) (layers "B.Cu" "B.Paste" "B.Mask") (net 3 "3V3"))
  (pad "117" smd rect (at -12.738 3.25 270) (size 0.3 1.475) (layers "B.Cu" "B.Paste" "B.Mask") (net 68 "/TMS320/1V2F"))
  (pad "118" smd rect (at -12.738 3.75 270) (size 0.3 1.475) (layers "B.Cu" "B.Paste" "B.Mask") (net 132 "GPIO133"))
  (pad "119" smd rect (at -12.738 4.25 270) (size 0.3 1.475) (layers "B.Cu" "B.Paste" "B.Mask") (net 3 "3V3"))
  (pad "120" smd rect (at -12.738 4.75 270) (size 0.3 1.475) (layers "B.Cu" "B.Paste" "B.Mask") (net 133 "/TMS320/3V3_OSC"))
  (pad "121" smd rect (at -12.738 5.25 270) (size 0.3 1.475) (layers "B.Cu" "B.Paste" "B.Mask") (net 7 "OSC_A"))
  (pad "122" smd rect (at -12.738 5.75 270) (size 0.3 1.475) (layers "B.Cu" "B.Paste" "B.Mask") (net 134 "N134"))
  (pad "123" smd rect (at -12.738 6.25 270) (size 0.3 1.475) (layers "B.Cu" "B.Paste" "B.Mask") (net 8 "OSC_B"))
  (pad "124" smd rect (at -12.738 6.75 270) (size 0.3 1.475) (layers "B.Cu" "B.Paste" "B.Mask") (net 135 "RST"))
  (pad "125" smd rect (at -12.738 7.25 270) (size 0.3 1.475) (layers "B.Cu" "B.Paste" "B.Mask") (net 133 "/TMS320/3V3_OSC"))
  (pad "126" smd rect (at -12.738 7.75 270) (size 0.3 1.475) (layers "B.Cu" "B.Paste" "B.Mask") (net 68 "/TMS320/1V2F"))
  (pad "127" smd rect (at -12.738 8.25 270) (size 0.3 1.475) (layers "B.Cu" "B.Paste" "B.Mask") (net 3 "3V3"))
  (pad "128" smd rect (at -12.738 8.75 270) (size 0.3 1.475) (layers "B.Cu" "B.Paste" "B.Mask") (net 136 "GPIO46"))
  (pad "129" smd rect (at -12.738 9.25 270) (size 0.3 1.475) (layers "B.Cu" "B.Paste" "B.Mask") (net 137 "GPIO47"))
  (pad "130" smd rect (at -12.738 9.75 270) (size 0.3 1.475) (layers "B.Cu" "B.Paste" "B.Mask") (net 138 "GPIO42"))
  (pad "131" smd rect (at -12.738 10.25 270) (size 0.3 1.475) (layers "B.Cu" "B.Paste" "B.Mask") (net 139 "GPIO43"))
  (pad "132" smd rect (at -12.738 10.75 270) (size 0.3 1.475) (layers "B.Cu" "B.Paste" "B.Mask") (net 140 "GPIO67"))
  (pad "133" smd rect (at -10.75 12.738 180) (size 0.3 1.475) (layers "B.Cu" "B.Paste" "B.Mask") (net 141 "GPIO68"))
  (pad "134" smd rect (at -10.25 12.738 180) (size 0.3 1.475) (layers "B.Cu" "B.Paste" "B.Mask") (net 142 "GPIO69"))
  (pad "135" smd rect (at -9.75 12.738 180) (size 0.3 1.475) (layers "B.Cu" "B.Paste" "B.Mask") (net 40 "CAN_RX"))
  (pad "136" smd rect (at -9.25 12.738 180) (size 0.3 1.475) (layers "B.Cu" "B.Paste" "B.Mask") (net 41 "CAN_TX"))
  (pad "137" smd rect (at -8.75 12.738 180) (size 0.3 1.475) (layers "B.Cu" "B.Paste" "B.Mask") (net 68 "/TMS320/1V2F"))
  (pad "138" smd rect (at -8.25 12.738 180) (size 0.3 1.475) (layers "B.Cu" "B.Paste" "B.Mask") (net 3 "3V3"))
  (pad "139" smd rect (at -7.75 12.738 180) (size 0.3 1.475) (layers "B.Cu" "B.Paste" "B.Mask") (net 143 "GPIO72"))
  (pad "140" smd rect (at -7.25 12.738 180) (size 0.3 1.475) (layers "B.Cu" "B.Paste" "B.Mask") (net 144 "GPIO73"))
  (pad "141" smd rect (at -6.75 12.738 180) (size 0.3 1.475) (layers "B.Cu" "B.Paste" "B.Mask") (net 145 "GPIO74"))
  (pad "142" smd rect (at -6.25 12.738 180) (size 0.3 1.475) (layers "B.Cu" "B.Paste" "B.Mask") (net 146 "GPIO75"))
  (pad "143" smd rect (at -5.75 12.738 180) (size 0.3 1.475) (layers "B.Cu" "B.Paste" "B.Mask") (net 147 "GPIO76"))
  (pad "144" smd rect (at -5.25 12.738 180) (size 0.3 1.475) (layers "B.Cu" "B.Paste" "B.Mask") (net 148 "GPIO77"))
  (pad "145" smd rect (at -4.75 12.738 180) (size 0.3 1.475) (layers "B.Cu" "B.Paste" "B.Mask") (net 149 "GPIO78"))
  (pad "146" smd rect (at -4.25 12.738 180) (size 0.3 1.475) (layers "B.Cu" "B.Paste" "B.Mask") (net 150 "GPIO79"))
  (pad "147" smd rect (at -3.75 12.738 180) (size 0.3 1.475) (layers "B.Cu" "B.Paste" "B.Mask") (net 3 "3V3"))
  (pad "148" smd rect (at -3.25 12.738 180) (size 0.3 1.475) (layers "B.Cu" "B.Paste" "B.Mask") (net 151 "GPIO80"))
  (pad "149" smd rect (at -2.75 12.738 180) (size 0.3 1.475) (layers "B.Cu" "B.Paste" "B.Mask") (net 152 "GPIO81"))
  (pad "150" smd rect (at -2.25 12.738 180) (size 0.3 1.475) (layers "B.Cu" "B.Paste" "B.Mask") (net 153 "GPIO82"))
  (pad "151" smd rect (at -1.75 12.738 180) (size 0.3 1.475) (layers "B.Cu" "B.Paste" "B.Mask") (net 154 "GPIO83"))
  (pad "152" smd rect (at -1.25 12.738 180) (size 0.3 1.475) (layers "B.Cu" "B.Paste" "B.Mask") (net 3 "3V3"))
  (pad "153" smd rect (at -0.75 12.738 180) (size 0.3 1.475) (layers "B.Cu" "B.Paste" "B.Mask") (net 68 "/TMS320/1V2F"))
  (pad "154" smd rect (at -0.25 12.738 180) (size 0.3 1.475) (layers "B.Cu" "B.Paste" "B.Mask") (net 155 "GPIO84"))
  (pad "155" smd rect (at 0.25 12.738 180) (size 0.3 1.475) (layers "B.Cu" "B.Paste" "B.Mask") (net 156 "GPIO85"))
  (pad "156" smd rect (at 0.75 12.738 180) (size 0.3 1.475) (layers "B.Cu" "B.Paste" "B.Mask") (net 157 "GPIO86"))
  (pad "157" smd rect (at 1.25 12.738 180) (size 0.3 1.475) (layers "B.Cu" "B.Paste" "B.Mask") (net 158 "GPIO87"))
  (pad "158" smd rect (at 1.75 12.738 180) (size 0.3 1.475) (layers "B.Cu" "B.Paste" "B.Mask") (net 68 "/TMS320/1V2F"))
  (pad "159" smd rect (at 2.25 12.738 180) (size 0.3 1.475) (layers "B.Cu" "B.Paste" "B.Mask") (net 3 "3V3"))
  (pad "160" smd rect (at 2.75 12.738 180) (size 0.3 1.475) (layers "B.Cu" "B.Paste" "B.Mask") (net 52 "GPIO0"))
  (pad "161" smd rect (at 3.25 12.738 180) (size 0.3 1.475) (layers "B.Cu" "B.Paste" "B.Mask") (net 49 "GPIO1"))
  (pad "162" smd rect (at 3.75 12.738 180) (size 0.3 1.475) (layers "B.Cu" "B.Paste" "B.Mask") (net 54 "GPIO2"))
  (pad "163" smd rect (at 4.25 12.738 180) (size 0.3 1.475) (layers "B.Cu" "B.Paste" "B.Mask") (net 50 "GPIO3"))
  (pad "164" smd rect (at 4.75 12.738 180) (size 0.3 1.475) (layers "B.Cu" "B.Paste" "B.Mask") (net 55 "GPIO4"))
  (pad "165" smd rect (at 5.25 12.738 180) (size 0.3 1.475) (layers "B.Cu" "B.Paste" "B.Mask") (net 51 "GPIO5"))
  (pad "166" smd rect (at 5.75 12.738 180) (size 0.3 1.475) (layers "B.Cu" "B.Paste" "B.Mask") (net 47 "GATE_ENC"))
  (pad "167" smd rect (at 6.25 12.738 180) (size 0.3 1.475) (layers "B.Cu" "B.Paste" "B.Mask") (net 46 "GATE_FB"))
  (pad "168" smd rect (at 6.75 12.738 180) (size 0.3 1.475) (layers "B.Cu" "B.Paste" "B.Mask") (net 3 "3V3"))
  (pad "169" smd rect (at 7.25 12.738 180) (size 0.3 1.475) (layers "B.Cu" "B.Paste" "B.Mask") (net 68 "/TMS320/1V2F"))
  (pad "170" smd rect (at 7.75 12.738 180) (size 0.3 1.475) (layers "B.Cu" "B.Paste" "B.Mask") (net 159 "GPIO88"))
  (pad "171" smd rect (at 8.25 12.738 180) (size 0.3 1.475) (layers "B.Cu" "B.Paste" "B.Mask") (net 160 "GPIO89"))
  (pad "172" smd rect (at 8.75 12.738 180) (size 0.3 1.475) (layers "B.Cu" "B.Paste" "B.Mask") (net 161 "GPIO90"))
  (pad "173" smd rect (at 9.25 12.738 180) (size 0.3 1.475) (layers "B.Cu" "B.Paste" "B.Mask") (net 38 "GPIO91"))
  (pad "174" smd rect (at 9.75 12.738 180) (size 0.3 1.475) (layers "B.Cu" "B.Paste" "B.Mask") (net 37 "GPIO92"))
  (pad "175" smd rect (at 10.25 12.738 180) (size 0.3 1.475) (layers "B.Cu" "B.Paste" "B.Mask") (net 44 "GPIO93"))
  (pad "176" smd rect (at 10.75 12.738 180) (size 0.3 1.475) (layers "B.Cu" "B.Paste" "B.Mask") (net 45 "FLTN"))
  (pad "177" smd rect (at 0 0 270) (size 7.33 8.07) (layers "B.Cu" "B.Paste" "B.Mask") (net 17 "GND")))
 (gr_rect (start 146.3 66.3) (end 173.7 93.7) (stroke (width 0.05) (type default)) (fill none) (layer "Edge.Cuts"))
 (segment (start 154.325 82.75) (end 153.05 82.75) (width 0.15) (layer "F.Cu") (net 41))
 (segment (start 153.05 82.75) (end 153 82.8) (width 0.15) (layer "F.Cu") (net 41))
 (via (at 153 82.8) (size 0.6) (drill 0.3) (layers "F.Cu" "B.Cu") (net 41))
 (segment (start 153 82.8) (end 153 78.425736) (width 0.15) (layer "B.Cu") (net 41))
 (segment (start 161.775 75.5) (end 169.25 68.025) (width 0.15) (layer "B.Cu") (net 41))
 (segment (start 169.25 68.025) (end 169.25 67.262) (width 0.15) (layer "B.Cu") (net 41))
 (segment (start 155.925736 75.5) (end 161.775 75.5) (width 0.15) (layer "B.Cu") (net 41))
 (segment (start 153 78.425736) (end 155.925736 75.5) (width 0.15) (layer "B.Cu") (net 41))
 (segment (start 155.35 82.25) (end 154.325 82.25) (width 0.15) (layer "F.Cu") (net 40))
 (segment (start 155.5 82.1) (end 155.35 82.25) (width 0.15) (layer "F.Cu") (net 40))
 (via (at 155.5 82.1) (size 0.6) (drill 0.3) (layers "F.Cu" "B.Cu") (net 40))
 (segment (start 155.5 76.35) (end 156.05 75.8) (width 0.15) (layer "B.Cu") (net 40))
 (segment (start 169.75 68.1495) (end 169.75 67.262) (width 0.15) (layer "B.Cu") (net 40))
 (segment (start 155.5 82.1) (end 155.5 76.35) (width 0.15) (layer "B.Cu") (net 40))
 (segment (start 156.05 75.8) (end 162.0995 75.8) (width 0.15) (layer "B.Cu") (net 40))
 (segment (start 162.0995 75.8) (end 169.75 68.1495) (width 0.15) (layer "B.Cu") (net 40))
 (segment (start 154.325 79.75) (end 153.550001 79.75) (width 0.15) (layer "F.Cu") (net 37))
 (segment (start 151.225 77.424999) (end 151.225 77.15) (width 0.15) (layer "F.Cu") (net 37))
 (segment (start 151.225 77.15) (end 150.175 76.1) (width 0.15) (layer "F.Cu") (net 37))
 (segment (start 153.550001 79.75) (end 151.225 77.424999) (width 0.15) (layer "F.Cu") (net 37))
 (via (at 150.175 76.1) (size 0.6) (drill 0.3) (layers "F.Cu" "B.Cu") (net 37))
 (segment (start 150.25 76.025) (end 150.25 67.262) (width 0.15) (layer "B.Cu") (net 37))
 (segment (start 150.175 76.1) (end 150.25 76.025) (width 0.15) (layer "B.Cu") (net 37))
 (segment (start 150.7 77.399999) (end 153.550001 80.25) (width 0.15) (layer "F.Cu") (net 38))
 (segment (start 153.550001 80.25) (end 154.325 80.25) (width 0.15) (layer "F.Cu") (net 38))
 (via (at 150.7 77.399999) (size 0.6) (drill 0.3) (layers "F.Cu" "B.Cu") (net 38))
 (segment (start 150.7 77.399999) (end 150.7 67.312) (width 0.15) (layer "B.Cu") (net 38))
 (segment (start 150.7 67.312) (end 150.75 67.262) (width 0.15) (layer "B.Cu") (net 38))
 (segment (start 151.55 81.75) (end 151.1 82.2) (width 0.15) (layer "F.Cu") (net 1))
 (segment (start 154.325 81.75) (end 151.55 81.75) (width 0.15) (layer "F.Cu") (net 1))
 (segment (start 152.25 81.25) (end 151.1 80.1) (width 0.15) (layer "F.Cu") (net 2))
 (segment (start 154.325 81.25) (end 152.25 81.25) (width 0.15) (layer "F.Cu") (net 2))
 (segment (start 171 77.199999) (end 171 74.8) (width 0.15) (layer "F.Cu") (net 7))
 (segment (start 166.449999 81.75) (end 171 77.199999) (width 0.15) (layer "F.Cu") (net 7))
 (segment (start 165.675 81.75) (end 166.449999 81.75) (width 0.15) (layer "F.Cu") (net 7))
 (via (at 171 74.8) (size 0.6) (drill 0.3) (layers "F.Cu" "B.Cu") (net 7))
 (segment (start 171 74.8) (end 171.05 74.75) (width 0.15) (layer "B.Cu") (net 7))
 (segment (start 171.05 74.75) (end 172.738 74.75) (width 0.15) (layer "B.Cu") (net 7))
 (segment (start 170.6 74) (end 170.475 74.125) (width 0.15) (layer "F.Cu") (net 8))
 (segment (start 170.475 77.2) (end 166.425 81.25) (width 0.15) (layer "F.Cu") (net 8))
 (segment (start 170.475 74.125) (end 170.475 77.2) (width 0.15) (layer "F.Cu") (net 8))
 (segment (start 166.425 81.25) (end 165.675 81.25) (width 0.15) (layer "F.Cu") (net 8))
 (via (at 170.6 74) (size 0.6) (drill 0.3) (layers "F.Cu" "B.Cu") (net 8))
 (segment (start 170.85 73.75) (end 170.6 74) (width 0.15) (layer "B.Cu") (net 8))
 (segment (start 172.738 73.75) (end 170.85 73.75) (width 0.15) (layer "B.Cu") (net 8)))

